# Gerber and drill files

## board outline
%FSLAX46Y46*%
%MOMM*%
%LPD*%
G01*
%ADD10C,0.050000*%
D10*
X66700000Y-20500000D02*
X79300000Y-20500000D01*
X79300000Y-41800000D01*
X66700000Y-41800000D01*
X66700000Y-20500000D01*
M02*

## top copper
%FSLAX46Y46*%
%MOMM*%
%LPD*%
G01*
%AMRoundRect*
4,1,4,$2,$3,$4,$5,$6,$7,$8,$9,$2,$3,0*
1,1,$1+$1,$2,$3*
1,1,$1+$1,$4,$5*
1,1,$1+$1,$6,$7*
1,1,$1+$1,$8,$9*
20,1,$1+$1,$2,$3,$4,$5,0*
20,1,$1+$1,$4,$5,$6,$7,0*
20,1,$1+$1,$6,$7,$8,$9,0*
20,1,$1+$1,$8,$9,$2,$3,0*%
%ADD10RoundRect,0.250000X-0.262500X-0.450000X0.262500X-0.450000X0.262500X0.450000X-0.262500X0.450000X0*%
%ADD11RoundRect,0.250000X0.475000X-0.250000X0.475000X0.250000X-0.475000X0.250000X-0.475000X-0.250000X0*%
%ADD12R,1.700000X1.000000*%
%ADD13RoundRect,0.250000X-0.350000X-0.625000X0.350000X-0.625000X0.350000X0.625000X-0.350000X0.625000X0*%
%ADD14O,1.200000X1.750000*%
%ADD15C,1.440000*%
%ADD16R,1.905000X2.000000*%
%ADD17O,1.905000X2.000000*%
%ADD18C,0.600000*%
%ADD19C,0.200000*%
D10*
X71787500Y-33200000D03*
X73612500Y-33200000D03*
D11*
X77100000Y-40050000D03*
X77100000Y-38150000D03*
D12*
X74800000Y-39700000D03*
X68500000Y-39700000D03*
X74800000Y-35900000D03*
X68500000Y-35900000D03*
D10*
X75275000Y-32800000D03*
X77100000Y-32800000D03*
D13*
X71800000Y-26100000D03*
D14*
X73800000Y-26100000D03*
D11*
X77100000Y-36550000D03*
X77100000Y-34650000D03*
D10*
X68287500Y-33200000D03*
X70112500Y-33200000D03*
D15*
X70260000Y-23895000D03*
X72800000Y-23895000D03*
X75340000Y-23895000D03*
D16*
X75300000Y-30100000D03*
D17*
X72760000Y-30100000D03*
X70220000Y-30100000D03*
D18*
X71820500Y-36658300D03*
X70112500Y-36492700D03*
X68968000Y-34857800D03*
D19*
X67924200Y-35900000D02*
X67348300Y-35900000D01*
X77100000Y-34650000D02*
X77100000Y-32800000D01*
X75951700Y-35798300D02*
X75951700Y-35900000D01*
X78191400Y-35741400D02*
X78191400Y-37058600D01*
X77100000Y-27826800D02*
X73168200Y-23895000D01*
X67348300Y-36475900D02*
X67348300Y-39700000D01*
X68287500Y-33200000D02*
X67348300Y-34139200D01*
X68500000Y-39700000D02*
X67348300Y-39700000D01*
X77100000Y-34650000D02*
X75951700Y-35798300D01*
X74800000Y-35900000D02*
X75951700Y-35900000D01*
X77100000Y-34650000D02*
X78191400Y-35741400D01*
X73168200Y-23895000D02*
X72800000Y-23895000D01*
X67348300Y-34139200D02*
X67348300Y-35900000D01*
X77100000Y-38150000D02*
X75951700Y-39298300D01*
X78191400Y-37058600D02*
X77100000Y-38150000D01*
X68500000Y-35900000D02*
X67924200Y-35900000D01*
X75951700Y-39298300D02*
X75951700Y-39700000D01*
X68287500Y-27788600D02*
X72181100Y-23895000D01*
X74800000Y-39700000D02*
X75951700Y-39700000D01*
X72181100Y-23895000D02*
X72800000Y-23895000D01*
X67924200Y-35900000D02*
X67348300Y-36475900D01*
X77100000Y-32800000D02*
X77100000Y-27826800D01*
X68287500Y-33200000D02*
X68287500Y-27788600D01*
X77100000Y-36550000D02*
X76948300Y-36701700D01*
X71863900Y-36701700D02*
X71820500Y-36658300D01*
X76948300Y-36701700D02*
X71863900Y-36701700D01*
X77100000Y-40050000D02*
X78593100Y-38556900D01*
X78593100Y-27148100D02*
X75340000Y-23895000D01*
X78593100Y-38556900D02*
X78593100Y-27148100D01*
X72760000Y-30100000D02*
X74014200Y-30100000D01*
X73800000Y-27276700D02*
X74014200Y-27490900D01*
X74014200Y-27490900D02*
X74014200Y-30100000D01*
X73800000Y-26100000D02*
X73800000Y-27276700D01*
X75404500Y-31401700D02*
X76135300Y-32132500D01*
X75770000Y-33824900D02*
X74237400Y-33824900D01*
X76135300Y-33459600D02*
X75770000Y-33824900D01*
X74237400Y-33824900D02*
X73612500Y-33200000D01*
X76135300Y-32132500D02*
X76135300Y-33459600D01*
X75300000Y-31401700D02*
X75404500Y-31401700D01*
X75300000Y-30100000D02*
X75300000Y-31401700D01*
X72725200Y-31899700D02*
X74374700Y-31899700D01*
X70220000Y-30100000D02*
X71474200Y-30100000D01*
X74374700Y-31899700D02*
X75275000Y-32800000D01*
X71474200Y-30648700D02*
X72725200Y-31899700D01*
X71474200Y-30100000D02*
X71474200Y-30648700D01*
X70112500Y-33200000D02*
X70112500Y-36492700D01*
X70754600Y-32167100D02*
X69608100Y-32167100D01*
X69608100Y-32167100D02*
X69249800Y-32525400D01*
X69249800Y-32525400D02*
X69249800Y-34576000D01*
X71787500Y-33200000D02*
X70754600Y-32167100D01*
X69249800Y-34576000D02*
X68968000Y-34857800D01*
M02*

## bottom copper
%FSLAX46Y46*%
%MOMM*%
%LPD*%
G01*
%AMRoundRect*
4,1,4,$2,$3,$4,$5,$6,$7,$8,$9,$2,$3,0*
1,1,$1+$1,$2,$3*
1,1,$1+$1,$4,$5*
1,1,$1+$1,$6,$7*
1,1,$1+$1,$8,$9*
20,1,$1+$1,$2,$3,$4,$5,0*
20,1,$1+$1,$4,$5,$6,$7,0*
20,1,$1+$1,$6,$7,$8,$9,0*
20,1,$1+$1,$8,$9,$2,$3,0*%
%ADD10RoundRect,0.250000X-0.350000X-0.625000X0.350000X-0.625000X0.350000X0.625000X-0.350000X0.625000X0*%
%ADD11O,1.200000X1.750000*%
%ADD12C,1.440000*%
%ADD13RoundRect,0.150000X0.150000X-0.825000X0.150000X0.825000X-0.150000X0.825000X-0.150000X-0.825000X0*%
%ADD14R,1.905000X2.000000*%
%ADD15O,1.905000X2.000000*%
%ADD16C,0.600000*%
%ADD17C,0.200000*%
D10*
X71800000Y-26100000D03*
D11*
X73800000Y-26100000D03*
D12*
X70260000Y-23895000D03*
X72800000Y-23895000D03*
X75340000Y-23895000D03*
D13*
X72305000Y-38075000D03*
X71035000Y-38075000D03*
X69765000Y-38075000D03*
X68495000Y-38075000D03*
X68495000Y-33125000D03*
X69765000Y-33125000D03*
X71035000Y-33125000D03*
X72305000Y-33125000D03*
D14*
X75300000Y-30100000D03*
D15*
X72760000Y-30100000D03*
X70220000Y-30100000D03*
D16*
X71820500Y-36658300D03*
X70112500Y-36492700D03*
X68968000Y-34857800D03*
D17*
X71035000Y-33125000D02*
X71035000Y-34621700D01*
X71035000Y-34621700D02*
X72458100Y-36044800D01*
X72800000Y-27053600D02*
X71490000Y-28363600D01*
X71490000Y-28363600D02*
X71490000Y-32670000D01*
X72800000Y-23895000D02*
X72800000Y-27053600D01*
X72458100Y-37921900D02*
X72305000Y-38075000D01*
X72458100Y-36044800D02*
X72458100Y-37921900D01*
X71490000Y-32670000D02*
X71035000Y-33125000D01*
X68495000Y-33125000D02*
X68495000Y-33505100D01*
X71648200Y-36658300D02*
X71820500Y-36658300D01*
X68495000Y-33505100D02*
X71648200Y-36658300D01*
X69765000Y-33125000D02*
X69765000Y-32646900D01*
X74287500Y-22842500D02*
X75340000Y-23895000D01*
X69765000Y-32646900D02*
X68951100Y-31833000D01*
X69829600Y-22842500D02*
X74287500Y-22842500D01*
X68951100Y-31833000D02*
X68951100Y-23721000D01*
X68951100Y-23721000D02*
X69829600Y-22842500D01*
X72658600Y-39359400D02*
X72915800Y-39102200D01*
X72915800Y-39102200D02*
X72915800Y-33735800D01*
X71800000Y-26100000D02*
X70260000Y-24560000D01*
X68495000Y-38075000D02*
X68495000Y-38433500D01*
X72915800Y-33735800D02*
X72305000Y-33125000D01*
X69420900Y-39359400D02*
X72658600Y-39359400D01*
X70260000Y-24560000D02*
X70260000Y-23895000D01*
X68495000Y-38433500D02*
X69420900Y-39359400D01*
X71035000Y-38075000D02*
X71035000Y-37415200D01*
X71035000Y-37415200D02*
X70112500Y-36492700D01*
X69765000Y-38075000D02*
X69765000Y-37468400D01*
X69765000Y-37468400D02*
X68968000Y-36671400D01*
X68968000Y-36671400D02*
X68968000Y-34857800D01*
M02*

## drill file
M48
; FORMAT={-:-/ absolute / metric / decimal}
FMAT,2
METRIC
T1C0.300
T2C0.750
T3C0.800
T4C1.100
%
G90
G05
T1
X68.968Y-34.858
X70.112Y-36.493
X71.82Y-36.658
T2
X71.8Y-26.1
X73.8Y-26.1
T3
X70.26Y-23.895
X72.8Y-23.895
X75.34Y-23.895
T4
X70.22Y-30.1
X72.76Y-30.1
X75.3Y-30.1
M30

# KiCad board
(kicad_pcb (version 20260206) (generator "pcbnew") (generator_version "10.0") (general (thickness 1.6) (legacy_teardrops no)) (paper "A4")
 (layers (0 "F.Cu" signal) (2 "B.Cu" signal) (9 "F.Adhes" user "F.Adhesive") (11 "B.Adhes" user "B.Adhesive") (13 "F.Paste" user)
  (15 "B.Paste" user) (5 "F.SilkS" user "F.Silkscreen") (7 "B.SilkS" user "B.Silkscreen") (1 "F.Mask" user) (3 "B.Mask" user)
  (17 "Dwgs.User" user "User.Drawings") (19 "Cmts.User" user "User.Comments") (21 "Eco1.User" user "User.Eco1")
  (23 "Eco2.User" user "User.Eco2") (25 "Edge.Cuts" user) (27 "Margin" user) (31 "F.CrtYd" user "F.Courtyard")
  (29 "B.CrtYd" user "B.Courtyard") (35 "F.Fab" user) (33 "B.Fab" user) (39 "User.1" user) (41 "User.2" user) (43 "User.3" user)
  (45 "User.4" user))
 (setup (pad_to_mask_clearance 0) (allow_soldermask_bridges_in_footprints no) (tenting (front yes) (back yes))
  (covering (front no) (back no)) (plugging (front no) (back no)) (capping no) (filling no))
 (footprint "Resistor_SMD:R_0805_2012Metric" (layer "F.Cu") (at 72.7 33.2)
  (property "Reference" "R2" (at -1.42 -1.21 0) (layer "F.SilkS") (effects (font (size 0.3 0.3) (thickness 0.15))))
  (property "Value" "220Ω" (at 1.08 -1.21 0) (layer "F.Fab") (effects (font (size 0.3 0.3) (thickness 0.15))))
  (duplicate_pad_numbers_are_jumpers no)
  (pad "1" smd roundrect (at -0.9125 0) (size 1.025 1.4) (layers "F.Cu" "F.Mask" "F.Paste") (roundrect_rratio 0.243902) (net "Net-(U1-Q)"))
  (pad "2" smd roundrect (at 0.9125 0) (size 1.025 1.4) (layers "F.Cu" "F.Mask" "F.Paste") (roundrect_rratio 0.243902) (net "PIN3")))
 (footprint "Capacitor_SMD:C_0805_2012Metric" (layer "F.Cu") (at 77.1 39.1 90)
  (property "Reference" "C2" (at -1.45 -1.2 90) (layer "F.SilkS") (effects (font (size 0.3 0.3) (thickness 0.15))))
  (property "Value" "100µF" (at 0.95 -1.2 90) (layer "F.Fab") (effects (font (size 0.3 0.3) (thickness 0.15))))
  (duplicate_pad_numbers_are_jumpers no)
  (pad "1" smd roundrect (at -0.95 0 90) (size 1 1.45) (layers "F.Cu" "F.Mask" "F.Paste") (roundrect_rratio 0.25) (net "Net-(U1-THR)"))
  (pad "2" smd roundrect (at 0.95 0 90) (size 1 1.45) (layers "F.Cu" "F.Mask" "F.Paste") (roundrect_rratio 0.25) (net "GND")))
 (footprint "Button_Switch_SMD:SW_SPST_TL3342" (layer "F.Cu") (at 71.65 37.8 180)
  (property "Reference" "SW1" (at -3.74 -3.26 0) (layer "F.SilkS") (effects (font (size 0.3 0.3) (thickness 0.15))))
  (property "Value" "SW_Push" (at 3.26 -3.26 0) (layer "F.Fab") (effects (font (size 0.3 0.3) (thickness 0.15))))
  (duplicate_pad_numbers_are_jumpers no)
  (pad "1" smd rect (at -3.15 -1.9 180) (size 1.7 1) (layers "F.Cu" "F.Mask" "F.Paste") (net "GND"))
  (pad "1" smd rect (at 3.15 -1.9 180) (size 1.7 1) (layers "F.Cu" "F.Mask" "F.Paste") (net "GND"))
  (pad "2" smd rect (at -3.15 1.9 180) (size 1.7 1) (layers "F.Cu" "F.Mask" "F.Paste") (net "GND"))
  (pad "2" smd rect (at 3.15 1.9 180) (size 1.7 1) (layers "F.Cu" "F.Mask" "F.Paste") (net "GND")))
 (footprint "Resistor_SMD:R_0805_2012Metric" (layer "F.Cu") (at 76.1875 32.8)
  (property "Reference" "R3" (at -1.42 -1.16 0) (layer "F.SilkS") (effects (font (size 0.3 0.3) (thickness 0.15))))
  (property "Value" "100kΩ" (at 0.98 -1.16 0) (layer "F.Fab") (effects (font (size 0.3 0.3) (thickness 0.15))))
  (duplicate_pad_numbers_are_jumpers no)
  (pad "1" smd roundrect (at -0.9125 0) (size 1.025 1.4) (layers "F.Cu" "F.Mask" "F.Paste") (roundrect_rratio 0.243902) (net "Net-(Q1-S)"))
  (pad "2" smd roundrect (at 0.9125 0) (size 1.025 1.4) (layers "F.Cu" "F.Mask" "F.Paste") (roundrect_rratio 0.243902) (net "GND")))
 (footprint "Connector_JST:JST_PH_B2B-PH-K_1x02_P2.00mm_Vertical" (layer "F.Cu") (at 71.8 26.1)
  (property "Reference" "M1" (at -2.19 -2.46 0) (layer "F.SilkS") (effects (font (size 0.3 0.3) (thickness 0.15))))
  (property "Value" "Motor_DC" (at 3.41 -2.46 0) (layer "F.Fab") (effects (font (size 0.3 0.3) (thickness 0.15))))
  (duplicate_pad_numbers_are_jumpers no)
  (pad "1" thru_hole roundrect (at 0 0) (size 1.2 1.75) (drill 0.75) (layers "*.Cu" "*.Mask") (remove_unused_layers no)
   (roundrect_rratio 0.208333) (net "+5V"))
  (pad "2" thru_hole oval (at 2 0) (size 1.2 1.75) (drill 0.75) (layers "*.Cu" "*.Mask") (remove_unused_layers no) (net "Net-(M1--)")))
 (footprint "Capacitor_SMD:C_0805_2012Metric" (layer "F.Cu") (at 77.1 35.6 90)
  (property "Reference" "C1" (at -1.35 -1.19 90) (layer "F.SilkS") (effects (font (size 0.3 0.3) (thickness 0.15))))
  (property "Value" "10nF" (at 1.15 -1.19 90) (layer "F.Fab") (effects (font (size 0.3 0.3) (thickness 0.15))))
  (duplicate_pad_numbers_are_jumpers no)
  (pad "1" smd roundrect (at -0.95 0 90) (size 1 1.45) (layers "F.Cu" "F.Mask" "F.Paste") (roundrect_rratio 0.25) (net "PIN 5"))
  (pad "2" smd roundrect (at 0.95 0 90) (size 1 1.45) (layers "F.Cu" "F.Mask" "F.Paste") (roundrect_rratio 0.25) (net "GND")))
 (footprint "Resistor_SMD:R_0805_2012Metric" (layer "F.Cu") (at 69.2 33.2)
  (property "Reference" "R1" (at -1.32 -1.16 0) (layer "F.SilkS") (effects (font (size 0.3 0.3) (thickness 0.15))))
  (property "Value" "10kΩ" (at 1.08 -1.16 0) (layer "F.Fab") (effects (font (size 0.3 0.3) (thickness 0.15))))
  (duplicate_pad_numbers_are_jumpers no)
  (pad "1" smd roundrect (at -0.9125 0) (size 1.025 1.4) (layers "F.Cu" "F.Mask" "F.Paste") (roundrect_rratio 0.243902) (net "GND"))
  (pad "2" smd roundrect (at 0.9125 0) (size 1.025 1.4) (layers "F.Cu" "F.Mask" "F.Paste") (roundrect_rratio 0.243902) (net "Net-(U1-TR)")))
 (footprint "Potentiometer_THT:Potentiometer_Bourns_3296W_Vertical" (layer "B.Cu") (at 70.26 23.895 180)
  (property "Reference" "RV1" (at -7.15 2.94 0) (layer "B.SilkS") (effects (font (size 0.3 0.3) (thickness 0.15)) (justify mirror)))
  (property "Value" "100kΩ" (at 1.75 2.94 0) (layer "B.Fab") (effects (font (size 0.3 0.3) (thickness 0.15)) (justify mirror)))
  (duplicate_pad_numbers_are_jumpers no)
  (pad "1" thru_hole circle (at 0 0 180) (size 1.44 1.44) (drill 0.8) (layers "*.Cu" "*.Mask") (remove_unused_layers no) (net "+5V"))
  (pad "2" thru_hole circle (at -2.54 0 180) (size 1.44 1.44) (drill 0.8) (layers "*.Cu" "*.Mask") (remove_unused_layers no) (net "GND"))
  (pad "3" thru_hole circle (at -5.08 0 180) (size 1.44 1.44) (drill 0.8) (layers "*.Cu" "*.Mask") (remove_unused_layers no)
   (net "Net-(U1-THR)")))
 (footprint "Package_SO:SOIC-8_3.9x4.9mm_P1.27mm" (layer "B.Cu") (at 70.4 35.6 90)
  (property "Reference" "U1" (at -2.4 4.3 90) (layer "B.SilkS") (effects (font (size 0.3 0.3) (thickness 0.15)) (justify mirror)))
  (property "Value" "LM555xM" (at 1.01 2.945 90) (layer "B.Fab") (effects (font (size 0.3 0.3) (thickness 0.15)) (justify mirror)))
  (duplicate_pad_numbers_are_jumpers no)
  (pad "1" smd roundrect (at -2.475 1.905 90) (size 1.95 0.6) (layers "B.Cu" "B.Mask" "B.Paste") (roundrect_rratio 0.25) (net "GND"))
  (pad "2" smd roundrect (at -2.475 0.635 90) (size 1.95 0.6) (layers "B.Cu" "B.Mask" "B.Paste") (roundrect_rratio 0.25) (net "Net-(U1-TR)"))
  (pad "3" smd roundrect (at -2.475 -0.635 90) (size 1.95 0.6) (layers "B.Cu" "B.Mask" "B.Paste") (roundrect_rratio 0.25) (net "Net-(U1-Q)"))
  (pad "4" smd roundrect (at -2.475 -1.905 90) (size 1.95 0.6) (layers "B.Cu" "B.Mask" "B.Paste") (roundrect_rratio 0.25) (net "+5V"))
  (pad "5" smd roundrect (at 2.475 -1.905 90) (size 1.95 0.6) (layers "B.Cu" "B.Mask" "B.Paste") (roundrect_rratio 0.25) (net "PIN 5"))
  (pad "6" smd roundrect (at 2.475 -0.635 90) (size 1.95 0.6) (layers "B.Cu" "B.Mask" "B.Paste") (roundrect_rratio 0.25)
   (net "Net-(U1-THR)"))
  (pad "7" smd roundrect (at 2.475 0.635 90) (size 1.95 0.6) (layers "B.Cu" "B.Mask" "B.Paste") (roundrect_rratio 0.25) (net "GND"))
  (pad "8" smd roundrect (at 2.475 1.905 90) (size 1.95 0.6) (layers "B.Cu" "B.Mask" "B.Paste") (roundrect_rratio 0.25) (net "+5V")))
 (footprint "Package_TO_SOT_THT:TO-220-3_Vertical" (layer "B.Cu") (at 75.3 30.1 180)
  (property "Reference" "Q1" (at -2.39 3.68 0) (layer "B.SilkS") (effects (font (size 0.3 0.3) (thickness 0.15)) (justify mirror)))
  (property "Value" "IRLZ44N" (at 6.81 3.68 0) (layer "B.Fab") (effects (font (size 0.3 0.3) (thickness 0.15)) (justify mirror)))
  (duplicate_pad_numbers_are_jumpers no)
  (pad "1" thru_hole rect (at 0 0 180) (size 1.905 2) (drill 1.1) (layers "*.Cu" "*.Mask") (remove_unused_layers no) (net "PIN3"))
  (pad "2" thru_hole oval (at 2.54 0 180) (size 1.905 2) (drill 1.1) (layers "*.Cu" "*.Mask") (remove_unused_layers no) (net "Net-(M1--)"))
  (pad "3" thru_hole oval (at 5.08 0 180) (size 1.905 2) (drill 1.1) (layers "*.Cu" "*.Mask") (remove_unused_layers no) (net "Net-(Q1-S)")))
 (gr_rect (start 66.7 20.5) (end 79.3 41.8) (stroke (width 0.05) (type default)) (fill no) (layer "Edge.Cuts"))
 (segment (start 67.9242 35.9) (end 67.3483 35.9) (width 0.2) (layer "F.Cu") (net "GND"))
 (segment (start 77.1 34.65) (end 77.1 32.8) (width 0.2) (layer "F.Cu") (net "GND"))
 (segment (start 75.9517 35.7983) (end 75.9517 35.9) (width 0.2) (layer "F.Cu") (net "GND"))
 (segment (start 78.1914 35.7414) (end 78.1914 37.0586) (width 0.2) (layer "F.Cu") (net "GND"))
 (segment (start 77.1 27.8268) (end 73.1682 23.895) (width 0.2) (layer "F.Cu") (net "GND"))
 (segment (start 67.3483 36.4759) (end 67.3483 39.7) (width 0.2) (layer "F.Cu") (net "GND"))
 (segment (start 68.2875 33.2) (end 67.3483 34.1392) (width 0.2) (layer "F.Cu") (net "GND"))
 (segment (start 68.5 39.7) (end 67.3483 39.7) (width 0.2) (layer "F.Cu") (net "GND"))
 (segment (start 77.1 34.65) (end 75.9517 35.7983) (width 0.2) (layer "F.Cu") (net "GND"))
 (segment (start 74.8 35.9) (end 75.9517 35.9) (width 0.2) (layer "F.Cu") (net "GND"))
 (segment (start 77.1 34.65) (end 78.1914 35.7414) (width 0.2) (layer "F.Cu") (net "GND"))
 (segment (start 73.1682 23.895) (end 72.8 23.895) (width 0.2) (layer "F.Cu") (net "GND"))
 (segment (start 67.3483 34.1392) (end 67.3483 35.9) (width 0.2) (layer "F.Cu") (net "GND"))
 (segment (start 77.1 38.15) (end 75.9517 39.2983) (width 0.2) (layer "F.Cu") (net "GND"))
 (segment (start 78.1914 37.0586) (end 77.1 38.15) (width 0.2) (layer "F.Cu") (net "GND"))
 (segment (start 68.5 35.9) (end 67.9242 35.9) (width 0.2) (layer "F.Cu") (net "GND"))
 (segment (start 75.9517 39.2983) (end 75.9517 39.7) (width 0.2) (layer "F.Cu") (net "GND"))
 (segment (start 68.2875 27.7886) (end 72.1811 23.895) (width 0.2) (layer "F.Cu") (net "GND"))
 (segment (start 74.8 39.7) (end 75.9517 39.7) (width 0.2) (layer "F.Cu") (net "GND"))
 (segment (start 72.1811 23.895) (end 72.8 23.895) (width 0.2) (layer "F.Cu") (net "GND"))
 (segment (start 67.9242 35.9) (end 67.3483 36.4759) (width 0.2) (layer "F.Cu") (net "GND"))
 (segment (start 77.1 32.8) (end 77.1 27.8268) (width 0.2) (layer "F.Cu") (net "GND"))
 (segment (start 68.2875 33.2) (end 68.2875 27.7886) (width 0.2) (layer "F.Cu") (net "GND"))
 (segment (start 71.035 33.125) (end 71.035 34.6217) (width 0.2) (layer "B.Cu") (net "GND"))
 (segment (start 71.035 34.6217) (end 72.4581 36.0448) (width 0.2) (layer "B.Cu") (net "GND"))
 (segment (start 72.8 27.0536) (end 71.49 28.3636) (width 0.2) (layer "B.Cu") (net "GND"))
 (segment (start 71.49 28.3636) (end 71.49 32.67) (width 0.2) (layer "B.Cu") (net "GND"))
 (segment (start 72.8 23.895) (end 72.8 27.0536) (width 0.2) (layer "B.Cu") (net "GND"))
 (segment (start 72.4581 37.9219) (end 72.305 38.075) (width 0.2) (layer "B.Cu") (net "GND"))
 (segment (start 72.4581 36.0448) (end 72.4581 37.9219) (width 0.2) (layer "B.Cu") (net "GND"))
 (segment (start 71.49 32.67) (end 71.035 33.125) (width 0.2) (layer "B.Cu") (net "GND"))
 (segment (start 77.1 36.55) (end 76.9483 36.7017) (width 0.2) (layer "F.Cu") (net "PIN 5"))
 (segment (start 71.8639 36.7017) (end 71.8205 36.6583) (width 0.2) (layer "F.Cu") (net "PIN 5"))
 (segment (start 76.9483 36.7017) (end 71.8639 36.7017) (width 0.2) (layer "F.Cu") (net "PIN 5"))
 (via (at 71.8205 36.6583) (size 0.6) (drill 0.3) (layers "F.Cu" "B.Cu") (capping no) (covering (front no) (back no))
  (plugging (front no) (back no)) (filling no) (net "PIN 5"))
 (segment (start 68.495 33.125) (end 68.495 33.5051) (width 0.2) (layer "B.Cu") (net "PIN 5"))
 (segment (start 71.6482 36.6583) (end 71.8205 36.6583) (width 0.2) (layer "B.Cu") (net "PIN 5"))
 (segment (start 68.495 33.5051) (end 71.6482 36.6583) (width 0.2) (layer "B.Cu") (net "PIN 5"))
 (segment (start 77.1 40.05) (end 78.5931 38.5569) (width 0.2) (layer "F.Cu") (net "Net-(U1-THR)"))
 (segment (start 78.5931 27.1481) (end 75.34 23.895) (width 0.2) (layer "F.Cu") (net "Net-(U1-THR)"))
 (segment (start 78.5931 38.5569) (end 78.5931 27.1481) (width 0.2) (layer "F.Cu") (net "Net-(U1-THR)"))
 (segment (start 69.765 33.125) (end 69.765 32.6469) (width 0.2) (layer "B.Cu") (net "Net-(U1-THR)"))
 (segment (start 74.2875 22.8425) (end 75.34 23.895) (width 0.2) (layer "B.Cu") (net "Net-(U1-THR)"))
 (segment (start 69.765 32.6469) (end 68.9511 31.833) (width 0.2) (layer "B.Cu") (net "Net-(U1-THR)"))
 (segment (start 69.8296 22.8425) (end 74.2875 22.8425) (width 0.2) (layer "B.Cu") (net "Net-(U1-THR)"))
 (segment (start 68.9511 31.833) (end 68.9511 23.721) (width 0.2) (layer "B.Cu") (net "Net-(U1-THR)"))
 (segment (start 68.9511 23.721) (end 69.8296 22.8425) (width 0.2) (layer "B.Cu") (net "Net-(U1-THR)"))
 (segment (start 72.76 30.1) (end 74.0142 30.1) (width 0.2) (layer "F.Cu") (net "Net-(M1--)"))
 (segment (start 73.8 27.2767) (end 74.0142 27.4909) (width 0.2) (layer "F.Cu") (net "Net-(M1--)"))
 (segment (start 74.0142 27.4909) (end 74.0142 30.1) (width 0.2) (layer "F.Cu") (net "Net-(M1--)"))
 (segment (start 73.8 26.1) (end 73.8 27.2767) (width 0.2) (layer "F.Cu") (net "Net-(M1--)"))
 (segment (start 72.6586 39.3594) (end 72.9158 39.1022) (width 0.2) (layer "B.Cu") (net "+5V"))
 (segment (start 72.9158 39.1022) (end 72.9158 33.7358) (width 0.2) (layer "B.Cu") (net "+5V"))
 (segment (start 71.8 26.1) (end 70.26 24.56) (width 0.2) (layer "B.Cu") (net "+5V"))
 (segment (start 68.495 38.075) (end 68.495 38.4335) (width 0.2) (layer "B.Cu") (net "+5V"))
 (segment (start 72.9158 33.7358) (end 72.305 33.125) (width 0.2) (layer "B.Cu") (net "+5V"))
 (segment (start 69.4209 39.3594) (end 72.6586 39.3594) (width 0.2) (layer "B.Cu") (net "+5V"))
 (segment (start 70.26 24.56) (end 70.26 23.895) (width 0.2) (layer "B.Cu") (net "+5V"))
 (segment (start 68.495 38.4335) (end 69.4209 39.3594) (width 0.2) (layer "B.Cu") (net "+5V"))
 (segment (start 75.4045 31.4017) (end 76.1353 32.1325) (width 0.2) (layer "F.Cu") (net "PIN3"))
 (segment (start 75.77 33.8249) (end 74.2374 33.8249) (width 0.2) (layer "F.Cu") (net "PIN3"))
 (segment (start 76.1353 33.4596) (end 75.77 33.8249) (width 0.2) (layer "F.Cu") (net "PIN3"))
 (segment (start 74.2374 33.8249) (end 73.6125 33.2) (width 0.2) (layer "F.Cu") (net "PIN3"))
 (segment (start 76.1353 32.1325) (end 76.1353 33.4596) (width 0.2) (layer "F.Cu") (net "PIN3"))
 (segment (start 75.3 31.4017) (end 75.4045 31.4017) (width 0.2) (layer "F.Cu") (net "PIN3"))
 (segment (start 75.3 30.1) (end 75.3 31.4017) (width 0.2) (layer "F.Cu") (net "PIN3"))
 (segment (start 72.7252 31.8997) (end 74.3747 31.8997) (width 0.2) (layer "F.Cu") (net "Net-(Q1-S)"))
 (segment (start 70.22 30.1) (end 71.4742 30.1) (width 0.2) (layer "F.Cu") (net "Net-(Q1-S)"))
 (segment (start 74.3747 31.8997) (end 75.275 32.8) (width 0.2) (layer "F.Cu") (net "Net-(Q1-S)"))
 (segment (start 71.4742 30.6487) (end 72.7252 31.8997) (width 0.2) (layer "F.Cu") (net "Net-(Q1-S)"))
 (segment (start 71.4742 30.1) (end 71.4742 30.6487) (width 0.2) (layer "F.Cu") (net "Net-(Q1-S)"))
 (segment (start 70.1125 33.2) (end 70.1125 36.4927) (width 0.2) (layer "F.Cu") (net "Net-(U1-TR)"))
 (via (at 70.1125 36.4927) (size 0.6) (drill 0.3) (layers "F.Cu" "B.Cu") (capping no) (covering (front no) (back no))
  (plugging (front no) (back no)) (filling no) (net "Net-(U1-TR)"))
 (segment (start 71.035 38.075) (end 71.035 37.4152) (width 0.2) (layer "B.Cu") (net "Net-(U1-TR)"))
 (segment (start 71.035 37.4152) (end 70.1125 36.4927) (width 0.2) (layer "B.Cu") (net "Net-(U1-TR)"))
 (segment (start 70.7546 32.1671) (end 69.6081 32.1671) (width 0.2) (layer "F.Cu") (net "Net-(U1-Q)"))
 (segment (start 69.6081 32.1671) (end 69.2498 32.5254) (width 0.2) (layer "F.Cu") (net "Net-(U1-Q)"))
 (segment (start 69.2498 32.5254) (end 69.2498 34.576) (width 0.2) (layer "F.Cu") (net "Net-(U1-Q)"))
 (segment (start 71.7875 33.2) (end 70.7546 32.1671) (width 0.2) (layer "F.Cu") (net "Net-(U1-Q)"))
 (segment (start 69.2498 34.576) (end 68.968 34.8578) (width 0.2) (layer "F.Cu") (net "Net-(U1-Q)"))
 (via (at 68.968 34.8578) (size 0.6) (drill 0.3) (layers "F.Cu" "B.Cu") (capping no) (covering (front no) (back no))
  (plugging (front no) (back no)) (filling no) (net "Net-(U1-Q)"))
 (segment (start 69.765 38.075) (end 69.765 37.4684) (width 0.2) (layer "B.Cu") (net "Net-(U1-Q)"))
 (segment (start 69.765 37.4684) (end 68.968 36.6714) (width 0.2) (layer "B.Cu") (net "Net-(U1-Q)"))
 (segment (start 68.968 36.6714) (end 68.968 34.8578) (width 0.2) (layer "B.Cu") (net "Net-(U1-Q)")))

